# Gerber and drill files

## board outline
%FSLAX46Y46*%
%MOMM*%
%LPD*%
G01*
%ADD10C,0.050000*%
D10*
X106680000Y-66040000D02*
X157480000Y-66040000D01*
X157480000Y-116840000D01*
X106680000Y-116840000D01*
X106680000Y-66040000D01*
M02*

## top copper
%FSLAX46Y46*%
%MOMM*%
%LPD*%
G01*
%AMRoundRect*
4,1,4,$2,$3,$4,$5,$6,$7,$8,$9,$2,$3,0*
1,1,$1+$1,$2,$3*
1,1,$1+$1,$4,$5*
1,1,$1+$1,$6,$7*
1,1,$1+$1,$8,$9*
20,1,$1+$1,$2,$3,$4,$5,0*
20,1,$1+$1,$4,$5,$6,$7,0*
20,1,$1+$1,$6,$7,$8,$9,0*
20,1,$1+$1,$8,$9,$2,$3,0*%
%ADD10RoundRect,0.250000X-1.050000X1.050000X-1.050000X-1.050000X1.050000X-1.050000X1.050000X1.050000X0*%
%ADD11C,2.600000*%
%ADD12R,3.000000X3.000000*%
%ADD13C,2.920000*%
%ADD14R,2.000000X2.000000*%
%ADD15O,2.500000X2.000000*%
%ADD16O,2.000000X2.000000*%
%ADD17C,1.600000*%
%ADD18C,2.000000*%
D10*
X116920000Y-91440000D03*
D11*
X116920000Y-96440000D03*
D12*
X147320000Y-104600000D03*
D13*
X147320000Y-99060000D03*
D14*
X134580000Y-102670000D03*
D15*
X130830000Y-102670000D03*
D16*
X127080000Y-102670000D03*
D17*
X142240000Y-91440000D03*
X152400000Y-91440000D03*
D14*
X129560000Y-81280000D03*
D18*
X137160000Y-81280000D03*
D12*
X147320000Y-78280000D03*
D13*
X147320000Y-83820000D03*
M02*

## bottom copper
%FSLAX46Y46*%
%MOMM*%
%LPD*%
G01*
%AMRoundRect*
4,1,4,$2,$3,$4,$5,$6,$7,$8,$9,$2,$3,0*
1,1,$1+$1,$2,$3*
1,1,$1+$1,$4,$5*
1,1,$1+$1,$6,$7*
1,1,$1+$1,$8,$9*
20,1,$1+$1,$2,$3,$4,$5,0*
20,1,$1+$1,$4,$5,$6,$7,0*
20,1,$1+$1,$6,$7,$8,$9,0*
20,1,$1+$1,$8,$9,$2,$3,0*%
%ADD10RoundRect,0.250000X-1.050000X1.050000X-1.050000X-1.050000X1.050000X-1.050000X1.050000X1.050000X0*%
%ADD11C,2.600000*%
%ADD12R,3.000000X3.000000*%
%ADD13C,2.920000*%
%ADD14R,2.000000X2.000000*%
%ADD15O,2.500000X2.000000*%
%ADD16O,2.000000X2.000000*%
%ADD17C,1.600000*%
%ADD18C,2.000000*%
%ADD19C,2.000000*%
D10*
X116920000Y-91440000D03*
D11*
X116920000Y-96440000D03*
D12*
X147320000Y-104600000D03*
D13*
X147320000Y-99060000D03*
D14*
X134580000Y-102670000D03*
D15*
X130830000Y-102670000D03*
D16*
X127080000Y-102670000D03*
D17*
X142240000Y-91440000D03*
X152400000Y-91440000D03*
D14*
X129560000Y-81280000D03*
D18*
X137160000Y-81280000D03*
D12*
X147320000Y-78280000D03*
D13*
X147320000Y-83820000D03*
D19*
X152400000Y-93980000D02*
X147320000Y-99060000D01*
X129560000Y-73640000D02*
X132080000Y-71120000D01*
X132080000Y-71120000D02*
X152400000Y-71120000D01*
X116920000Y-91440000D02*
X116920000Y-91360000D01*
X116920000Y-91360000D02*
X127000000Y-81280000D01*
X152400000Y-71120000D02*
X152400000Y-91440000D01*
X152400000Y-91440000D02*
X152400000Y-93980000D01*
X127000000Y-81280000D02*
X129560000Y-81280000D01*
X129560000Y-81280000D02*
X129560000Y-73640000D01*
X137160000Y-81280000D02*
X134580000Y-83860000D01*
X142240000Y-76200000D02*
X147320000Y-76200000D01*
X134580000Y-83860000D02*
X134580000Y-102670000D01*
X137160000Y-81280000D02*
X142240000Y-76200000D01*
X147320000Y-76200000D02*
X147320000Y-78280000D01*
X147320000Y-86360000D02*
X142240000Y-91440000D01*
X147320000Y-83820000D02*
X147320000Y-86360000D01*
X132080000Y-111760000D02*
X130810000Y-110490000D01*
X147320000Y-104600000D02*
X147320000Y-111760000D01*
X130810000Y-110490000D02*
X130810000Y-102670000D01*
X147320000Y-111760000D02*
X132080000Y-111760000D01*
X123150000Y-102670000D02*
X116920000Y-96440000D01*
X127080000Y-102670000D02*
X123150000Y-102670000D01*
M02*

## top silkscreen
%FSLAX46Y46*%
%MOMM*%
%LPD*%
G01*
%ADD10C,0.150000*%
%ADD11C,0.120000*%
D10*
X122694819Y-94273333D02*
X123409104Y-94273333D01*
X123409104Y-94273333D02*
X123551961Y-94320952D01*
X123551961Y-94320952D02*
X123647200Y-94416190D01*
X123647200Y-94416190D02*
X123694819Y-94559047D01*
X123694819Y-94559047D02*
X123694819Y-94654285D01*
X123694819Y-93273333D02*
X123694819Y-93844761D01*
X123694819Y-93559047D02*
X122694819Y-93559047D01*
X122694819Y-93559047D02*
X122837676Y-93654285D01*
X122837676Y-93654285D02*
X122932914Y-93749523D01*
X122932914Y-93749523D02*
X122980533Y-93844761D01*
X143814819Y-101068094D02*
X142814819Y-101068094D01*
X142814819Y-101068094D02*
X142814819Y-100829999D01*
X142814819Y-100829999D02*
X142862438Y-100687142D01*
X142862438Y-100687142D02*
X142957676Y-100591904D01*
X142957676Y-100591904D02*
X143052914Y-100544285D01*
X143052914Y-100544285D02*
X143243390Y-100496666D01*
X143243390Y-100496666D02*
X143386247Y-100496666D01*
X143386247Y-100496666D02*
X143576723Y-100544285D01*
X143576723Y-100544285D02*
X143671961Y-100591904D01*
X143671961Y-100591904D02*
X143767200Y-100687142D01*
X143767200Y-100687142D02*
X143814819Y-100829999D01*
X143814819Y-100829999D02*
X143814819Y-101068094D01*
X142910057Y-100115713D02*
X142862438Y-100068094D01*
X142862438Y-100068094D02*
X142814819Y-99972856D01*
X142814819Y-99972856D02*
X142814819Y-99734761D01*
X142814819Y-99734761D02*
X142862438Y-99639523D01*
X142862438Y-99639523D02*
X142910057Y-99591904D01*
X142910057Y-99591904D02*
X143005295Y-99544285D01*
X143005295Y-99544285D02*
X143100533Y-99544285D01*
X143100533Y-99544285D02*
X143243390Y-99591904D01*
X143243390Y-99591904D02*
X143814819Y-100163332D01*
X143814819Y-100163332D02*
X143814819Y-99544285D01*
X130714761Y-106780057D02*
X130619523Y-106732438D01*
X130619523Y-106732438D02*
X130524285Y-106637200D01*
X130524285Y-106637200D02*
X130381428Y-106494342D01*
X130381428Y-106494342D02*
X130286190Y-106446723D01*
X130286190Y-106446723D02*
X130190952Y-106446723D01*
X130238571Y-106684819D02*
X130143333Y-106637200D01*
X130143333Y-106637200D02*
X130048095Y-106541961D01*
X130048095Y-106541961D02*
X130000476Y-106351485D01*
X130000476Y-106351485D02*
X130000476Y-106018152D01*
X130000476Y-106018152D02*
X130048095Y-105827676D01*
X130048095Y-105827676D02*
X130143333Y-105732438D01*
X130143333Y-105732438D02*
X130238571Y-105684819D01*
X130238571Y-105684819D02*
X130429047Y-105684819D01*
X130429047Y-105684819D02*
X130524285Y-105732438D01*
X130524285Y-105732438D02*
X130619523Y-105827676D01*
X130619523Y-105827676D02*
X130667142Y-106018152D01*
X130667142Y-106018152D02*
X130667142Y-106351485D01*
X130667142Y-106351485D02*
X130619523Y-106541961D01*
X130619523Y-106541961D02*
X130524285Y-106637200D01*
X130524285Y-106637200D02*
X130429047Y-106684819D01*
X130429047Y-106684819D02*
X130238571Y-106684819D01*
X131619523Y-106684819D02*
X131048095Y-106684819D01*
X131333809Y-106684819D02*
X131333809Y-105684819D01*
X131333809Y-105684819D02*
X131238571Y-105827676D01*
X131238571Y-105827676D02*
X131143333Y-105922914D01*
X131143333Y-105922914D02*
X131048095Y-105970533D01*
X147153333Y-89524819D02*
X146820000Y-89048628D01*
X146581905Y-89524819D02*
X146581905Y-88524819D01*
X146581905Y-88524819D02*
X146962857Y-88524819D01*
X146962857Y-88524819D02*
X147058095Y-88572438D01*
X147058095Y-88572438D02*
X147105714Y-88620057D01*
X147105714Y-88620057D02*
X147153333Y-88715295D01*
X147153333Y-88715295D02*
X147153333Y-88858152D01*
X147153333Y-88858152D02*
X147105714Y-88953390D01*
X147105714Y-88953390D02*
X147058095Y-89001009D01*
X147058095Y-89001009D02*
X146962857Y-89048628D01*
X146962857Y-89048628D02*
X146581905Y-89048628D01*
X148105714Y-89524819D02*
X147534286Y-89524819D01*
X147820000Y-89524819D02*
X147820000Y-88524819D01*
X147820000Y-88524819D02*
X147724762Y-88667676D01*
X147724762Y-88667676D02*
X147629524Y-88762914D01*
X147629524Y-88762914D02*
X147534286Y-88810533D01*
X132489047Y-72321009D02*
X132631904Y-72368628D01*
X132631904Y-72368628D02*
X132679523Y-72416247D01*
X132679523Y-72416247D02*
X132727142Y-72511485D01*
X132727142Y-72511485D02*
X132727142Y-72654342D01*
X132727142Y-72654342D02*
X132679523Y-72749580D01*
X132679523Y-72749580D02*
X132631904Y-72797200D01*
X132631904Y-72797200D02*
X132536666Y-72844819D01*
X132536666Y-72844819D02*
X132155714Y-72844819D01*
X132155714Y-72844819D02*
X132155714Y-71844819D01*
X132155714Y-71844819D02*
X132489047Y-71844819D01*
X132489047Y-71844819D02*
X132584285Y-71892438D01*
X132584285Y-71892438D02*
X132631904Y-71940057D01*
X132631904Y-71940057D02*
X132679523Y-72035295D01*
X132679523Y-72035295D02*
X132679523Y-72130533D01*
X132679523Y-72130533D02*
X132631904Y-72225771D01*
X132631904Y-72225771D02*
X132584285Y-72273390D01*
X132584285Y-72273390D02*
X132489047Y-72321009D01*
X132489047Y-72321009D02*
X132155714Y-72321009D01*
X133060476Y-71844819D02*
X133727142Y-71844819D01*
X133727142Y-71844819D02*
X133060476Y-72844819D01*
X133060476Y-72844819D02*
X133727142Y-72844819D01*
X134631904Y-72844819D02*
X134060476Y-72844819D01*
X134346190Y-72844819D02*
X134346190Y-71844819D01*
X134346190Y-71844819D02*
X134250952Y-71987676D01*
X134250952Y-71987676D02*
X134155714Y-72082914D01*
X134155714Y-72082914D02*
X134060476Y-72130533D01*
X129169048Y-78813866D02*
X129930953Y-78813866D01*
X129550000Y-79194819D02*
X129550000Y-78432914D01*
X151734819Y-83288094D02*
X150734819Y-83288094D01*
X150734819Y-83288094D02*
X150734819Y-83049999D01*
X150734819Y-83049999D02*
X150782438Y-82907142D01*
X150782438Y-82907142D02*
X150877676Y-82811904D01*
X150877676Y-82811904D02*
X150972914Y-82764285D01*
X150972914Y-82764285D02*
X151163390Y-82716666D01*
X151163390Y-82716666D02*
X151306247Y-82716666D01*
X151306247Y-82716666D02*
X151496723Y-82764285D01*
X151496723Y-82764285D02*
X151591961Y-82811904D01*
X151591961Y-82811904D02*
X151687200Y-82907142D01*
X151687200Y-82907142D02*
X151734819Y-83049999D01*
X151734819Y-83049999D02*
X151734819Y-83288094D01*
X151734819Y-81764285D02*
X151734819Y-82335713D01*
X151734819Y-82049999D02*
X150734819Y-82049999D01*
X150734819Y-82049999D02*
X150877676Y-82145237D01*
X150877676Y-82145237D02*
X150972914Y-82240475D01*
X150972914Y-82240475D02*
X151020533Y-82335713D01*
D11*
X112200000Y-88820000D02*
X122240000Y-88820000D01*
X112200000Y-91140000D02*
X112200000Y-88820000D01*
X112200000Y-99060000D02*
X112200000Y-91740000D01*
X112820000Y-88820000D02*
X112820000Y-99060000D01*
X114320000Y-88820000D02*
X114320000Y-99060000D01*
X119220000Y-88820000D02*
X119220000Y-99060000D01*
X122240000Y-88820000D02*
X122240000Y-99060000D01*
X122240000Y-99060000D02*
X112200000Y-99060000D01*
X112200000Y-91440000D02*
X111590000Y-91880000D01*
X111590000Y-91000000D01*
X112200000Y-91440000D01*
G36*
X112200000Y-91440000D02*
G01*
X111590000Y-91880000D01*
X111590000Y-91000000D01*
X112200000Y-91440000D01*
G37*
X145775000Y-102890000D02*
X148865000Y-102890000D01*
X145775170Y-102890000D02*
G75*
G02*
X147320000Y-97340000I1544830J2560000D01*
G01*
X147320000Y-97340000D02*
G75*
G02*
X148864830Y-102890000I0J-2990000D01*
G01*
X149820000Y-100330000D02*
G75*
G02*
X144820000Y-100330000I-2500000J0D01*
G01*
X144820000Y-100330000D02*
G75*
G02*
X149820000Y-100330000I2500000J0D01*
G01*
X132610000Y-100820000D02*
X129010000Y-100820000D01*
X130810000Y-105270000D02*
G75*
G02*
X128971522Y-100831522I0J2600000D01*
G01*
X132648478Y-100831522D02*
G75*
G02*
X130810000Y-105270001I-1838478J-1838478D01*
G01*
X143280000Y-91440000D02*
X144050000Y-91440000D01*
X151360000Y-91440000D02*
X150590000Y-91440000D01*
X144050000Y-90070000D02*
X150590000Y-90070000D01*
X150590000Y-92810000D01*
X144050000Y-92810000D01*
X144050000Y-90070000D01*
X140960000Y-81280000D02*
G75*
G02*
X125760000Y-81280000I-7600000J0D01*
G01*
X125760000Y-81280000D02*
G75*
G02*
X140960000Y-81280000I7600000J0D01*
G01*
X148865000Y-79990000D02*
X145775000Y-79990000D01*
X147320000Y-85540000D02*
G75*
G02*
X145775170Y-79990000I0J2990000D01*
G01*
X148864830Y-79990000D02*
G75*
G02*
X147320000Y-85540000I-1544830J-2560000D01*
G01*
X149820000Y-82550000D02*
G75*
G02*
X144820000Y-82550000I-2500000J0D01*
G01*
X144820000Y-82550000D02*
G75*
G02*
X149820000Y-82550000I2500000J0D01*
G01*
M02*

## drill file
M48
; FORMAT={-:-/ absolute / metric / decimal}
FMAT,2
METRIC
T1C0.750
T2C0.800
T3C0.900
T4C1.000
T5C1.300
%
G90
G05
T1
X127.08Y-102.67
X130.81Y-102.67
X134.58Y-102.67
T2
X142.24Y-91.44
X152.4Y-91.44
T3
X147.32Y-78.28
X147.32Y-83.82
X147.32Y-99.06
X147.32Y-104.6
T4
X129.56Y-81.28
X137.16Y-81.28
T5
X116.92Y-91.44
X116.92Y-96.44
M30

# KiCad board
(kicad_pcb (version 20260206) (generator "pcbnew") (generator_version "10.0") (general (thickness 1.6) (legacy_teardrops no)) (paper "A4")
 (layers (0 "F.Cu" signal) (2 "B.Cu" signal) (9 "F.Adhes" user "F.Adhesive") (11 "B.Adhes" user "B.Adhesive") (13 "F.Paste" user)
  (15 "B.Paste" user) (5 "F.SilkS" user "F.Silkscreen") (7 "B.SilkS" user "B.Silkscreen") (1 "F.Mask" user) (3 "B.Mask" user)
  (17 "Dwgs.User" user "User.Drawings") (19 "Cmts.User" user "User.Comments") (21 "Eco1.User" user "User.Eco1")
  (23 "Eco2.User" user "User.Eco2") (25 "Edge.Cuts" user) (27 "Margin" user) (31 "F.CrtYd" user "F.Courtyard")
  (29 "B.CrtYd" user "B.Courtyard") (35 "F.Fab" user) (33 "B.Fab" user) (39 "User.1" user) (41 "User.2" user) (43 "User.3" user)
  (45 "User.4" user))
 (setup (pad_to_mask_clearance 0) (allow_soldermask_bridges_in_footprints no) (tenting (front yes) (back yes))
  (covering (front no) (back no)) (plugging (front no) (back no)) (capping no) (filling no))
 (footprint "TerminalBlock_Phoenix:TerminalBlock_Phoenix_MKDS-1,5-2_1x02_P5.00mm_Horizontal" (layer "F.Cu") (at 116.92 91.44 -90)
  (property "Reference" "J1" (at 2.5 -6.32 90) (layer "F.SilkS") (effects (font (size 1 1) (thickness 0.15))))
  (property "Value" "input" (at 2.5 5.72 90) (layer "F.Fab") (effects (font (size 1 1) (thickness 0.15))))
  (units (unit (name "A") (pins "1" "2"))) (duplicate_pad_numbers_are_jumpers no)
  (fp_line (start -2.62 4.72) (end -2.62 -5.32) (stroke (width 0.12) (type solid)) (layer "F.SilkS"))
  (fp_line (start -0.3 4.72) (end -2.62 4.72) (stroke (width 0.12) (type solid)) (layer "F.SilkS"))
  (fp_line (start 7.62 4.72) (end 0.3 4.72) (stroke (width 0.12) (type solid)) (layer "F.SilkS"))
  (fp_line (start -2.62 4.1) (end 7.62 4.1) (stroke (width 0.12) (type solid)) (layer "F.SilkS"))
  (fp_line (start -2.62 2.6) (end 7.62 2.6) (stroke (width 0.12) (type solid)) (layer "F.SilkS"))
  (fp_line (start -2.62 -2.3) (end 7.62 -2.3) (stroke (width 0.12) (type solid)) (layer "F.SilkS"))
  (fp_line (start -2.62 -5.32) (end 7.62 -5.32) (stroke (width 0.12) (type solid)) (layer "F.SilkS"))
  (fp_line (start 7.62 -5.32) (end 7.62 4.72) (stroke (width 0.12) (type solid)) (layer "F.SilkS"))
  (fp_poly (pts (xy 0 4.72) (xy 0.44 5.33) (xy -0.44 5.33)) (stroke (width 0.12) (type solid)) (fill yes) (layer "F.SilkS"))
  (pad "1" thru_hole roundrect (at 0 0 270) (size 2.6 2.6) (drill 1.3) (layers "*.Cu" "*.Mask") (remove_unused_layers no)
   (roundrect_rratio 0.096154) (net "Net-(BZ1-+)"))
  (pad "2" thru_hole circle (at 5 0 270) (size 2.6 2.6) (drill 1.3) (layers "*.Cu" "*.Mask") (remove_unused_layers no)
   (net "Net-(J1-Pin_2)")))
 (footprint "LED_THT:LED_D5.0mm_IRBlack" (layer "F.Cu") (at 147.32 101.6 90)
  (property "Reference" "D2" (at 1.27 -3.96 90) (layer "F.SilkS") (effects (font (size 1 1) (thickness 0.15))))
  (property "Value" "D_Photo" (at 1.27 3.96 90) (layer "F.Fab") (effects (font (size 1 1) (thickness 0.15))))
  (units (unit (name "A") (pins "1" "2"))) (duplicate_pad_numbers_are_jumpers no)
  (fp_line (start -1.29 -1.545) (end -1.29 1.545) (stroke (width 0.12) (type solid)) (layer "F.SilkS"))
  (fp_arc (start -1.29 -1.54483) (mid 2.071779 -2.880495) (end 4.26 0) (stroke (width 0.12) (type solid)) (layer "F.SilkS"))
  (fp_arc (start 4.26 0) (mid 2.071779 2.880495) (end -1.29 1.54483) (stroke (width 0.12) (type solid)) (layer "F.SilkS"))
  (fp_circle (center 1.27 0) (end 3.77 0) (stroke (width 0.12) (type solid)) (fill no) (layer "F.SilkS"))
  (pad "1" thru_hole rect (at -3 0 90) (size 3 3) (drill 0.9) (layers "*.Cu" "*.Mask") (remove_unused_layers no) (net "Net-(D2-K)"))
  (pad "2" thru_hole circle (at 2.54 0 90) (size 2.92 2.92) (drill 0.9) (layers "*.Cu" "*.Mask") (remove_unused_layers no)
   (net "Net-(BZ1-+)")))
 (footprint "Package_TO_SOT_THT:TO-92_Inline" (layer "F.Cu") (at 132.08 102.67 180)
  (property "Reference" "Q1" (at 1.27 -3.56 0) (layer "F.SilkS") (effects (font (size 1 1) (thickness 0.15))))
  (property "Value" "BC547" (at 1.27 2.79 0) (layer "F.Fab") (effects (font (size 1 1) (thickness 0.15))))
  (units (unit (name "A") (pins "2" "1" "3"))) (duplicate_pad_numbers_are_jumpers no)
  (fp_line (start -0.53 1.85) (end 3.07 1.85) (stroke (width 0.12) (type solid)) (layer "F.SilkS"))
  (fp_arc (start 1.27 -2.6) (mid 3.672087 -0.994977) (end 3.108478 1.838478) (stroke (width 0.12) (type solid)) (layer "F.SilkS"))
  (fp_arc (start -0.568478 1.838478) (mid -1.132087 -0.994977) (end 1.27 -2.6) (stroke (width 0.12) (type solid)) (layer "F.SilkS"))
  (pad "1" thru_hole rect (at -2.5 0 180) (size 2 2) (drill 0.75) (layers "*.Cu" "*.Mask") (remove_unused_layers no) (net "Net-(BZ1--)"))
  (pad "2" thru_hole oval (at 1.27 0 180) (size 2.5 2) (drill 0.75 (offset -0.02 0)) (layers "*.Cu" "*.Mask") (remove_unused_layers no)
   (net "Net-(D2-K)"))
  (pad "3" thru_hole oval (at 5 0 180) (size 2 2) (drill 0.75) (layers "*.Cu" "*.Mask") (remove_unused_layers no) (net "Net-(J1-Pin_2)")))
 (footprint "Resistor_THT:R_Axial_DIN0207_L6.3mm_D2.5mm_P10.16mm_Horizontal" (layer "F.Cu") (at 142.24 91.44)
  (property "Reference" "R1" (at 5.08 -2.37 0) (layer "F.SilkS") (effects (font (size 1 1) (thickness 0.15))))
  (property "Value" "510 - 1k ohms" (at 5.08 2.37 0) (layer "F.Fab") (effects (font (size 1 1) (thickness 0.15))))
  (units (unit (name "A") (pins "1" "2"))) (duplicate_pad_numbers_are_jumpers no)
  (fp_line (start 1.04 0) (end 1.81 0) (stroke (width 0.12) (type solid)) (layer "F.SilkS"))
  (fp_line (start 9.12 0) (end 8.35 0) (stroke (width 0.12) (type solid)) (layer "F.SilkS"))
  (fp_rect (start 1.81 -1.37) (end 8.35 1.37) (stroke (width 0.12) (type solid)) (fill no) (layer "F.SilkS"))
  (pad "1" thru_hole circle (at 0 0) (size 1.6 1.6) (drill 0.8) (layers "*.Cu" "*.Mask") (remove_unused_layers no) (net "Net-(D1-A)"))
  (pad "2" thru_hole circle (at 10.16 0) (size 1.6 1.6) (drill 0.8) (layers "*.Cu" "*.Mask") (remove_unused_layers no) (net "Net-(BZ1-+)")))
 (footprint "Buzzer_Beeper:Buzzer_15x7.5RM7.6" (layer "F.Cu") (at 129.56 81.28)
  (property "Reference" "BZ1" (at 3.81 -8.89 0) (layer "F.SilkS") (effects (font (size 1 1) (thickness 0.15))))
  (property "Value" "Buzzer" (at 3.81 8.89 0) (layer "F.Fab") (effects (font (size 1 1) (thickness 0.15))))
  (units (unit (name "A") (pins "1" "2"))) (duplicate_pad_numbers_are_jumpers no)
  (fp_circle (center 3.8 0) (end 11.4 0) (stroke (width 0.12) (type solid)) (fill no) (layer "F.SilkS"))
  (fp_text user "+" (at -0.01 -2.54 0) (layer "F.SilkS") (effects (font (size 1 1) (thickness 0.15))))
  (pad "1" thru_hole rect (at 0 0) (size 2 2) (drill 1) (layers "*.Cu" "*.Mask") (remove_unused_layers no) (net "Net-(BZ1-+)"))
  (pad "2" thru_hole circle (at 7.6 0) (size 2 2) (drill 1) (layers "*.Cu" "*.Mask") (remove_unused_layers no) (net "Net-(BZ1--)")))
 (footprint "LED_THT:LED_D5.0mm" (layer "F.Cu") (at 147.32 81.28 -90)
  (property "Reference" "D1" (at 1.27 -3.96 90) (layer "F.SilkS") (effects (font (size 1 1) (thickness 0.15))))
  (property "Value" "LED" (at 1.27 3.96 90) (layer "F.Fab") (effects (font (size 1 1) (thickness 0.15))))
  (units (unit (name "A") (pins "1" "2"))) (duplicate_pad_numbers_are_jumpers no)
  (fp_line (start -1.29 -1.545) (end -1.29 1.545) (stroke (width 0.12) (type solid)) (layer "F.SilkS"))
  (fp_arc (start 4.26 0) (mid 2.071779 2.880495) (end -1.29 1.54483) (stroke (width 0.12) (type solid)) (layer "F.SilkS"))
  (fp_arc (start -1.29 -1.54483) (mid 2.071779 -2.880495) (end 4.26 0) (stroke (width 0.12) (type solid)) (layer "F.SilkS"))
  (fp_circle (center 1.27 0) (end 3.77 0) (stroke (width 0.12) (type solid)) (fill no) (layer "F.SilkS"))
  (pad "1" thru_hole rect (at -3 0 270) (size 3 3) (drill 0.9) (layers "*.Cu" "*.Mask") (remove_unused_layers no) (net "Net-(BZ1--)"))
  (pad "2" thru_hole circle (at 2.54 0 270) (size 2.92 2.92) (drill 0.9) (layers "*.Cu" "*.Mask") (remove_unused_layers no)
   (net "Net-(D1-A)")))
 (gr_rect (start 106.68 66.04) (end 157.48 116.84) (stroke (width 0.05) (type default)) (fill no) (layer "Edge.Cuts"))
 (segment (start 152.4 93.98) (end 147.32 99.06) (width 2) (layer "B.Cu") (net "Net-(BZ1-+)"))
 (segment (start 129.56 73.64) (end 132.08 71.12) (width 2) (layer "B.Cu") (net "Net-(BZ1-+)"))
 (segment (start 132.08 71.12) (end 152.4 71.12) (width 2) (layer "B.Cu") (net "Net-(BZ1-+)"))
 (segment (start 116.92 91.44) (end 116.92 91.36) (width 2) (layer "B.Cu") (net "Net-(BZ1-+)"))
 (segment (start 116.92 91.36) (end 127 81.28) (width 2) (layer "B.Cu") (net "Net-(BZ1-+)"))
 (segment (start 152.4 71.12) (end 152.4 91.44) (width 2) (layer "B.Cu") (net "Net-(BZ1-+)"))
 (segment (start 152.4 91.44) (end 152.4 93.98) (width 2) (layer "B.Cu") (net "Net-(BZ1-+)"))
 (segment (start 127 81.28) (end 129.56 81.28) (width 2) (layer "B.Cu") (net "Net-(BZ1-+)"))
 (segment (start 129.56 81.28) (end 129.56 73.64) (width 2) (layer "B.Cu") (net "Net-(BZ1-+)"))
 (segment (start 137.16 81.28) (end 134.58 83.86) (width 2) (layer "B.Cu") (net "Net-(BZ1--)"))
 (segment (start 142.24 76.2) (end 147.32 76.2) (width 2) (layer "B.Cu") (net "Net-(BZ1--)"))
 (segment (start 134.58 83.86) (end 134.58 102.67) (width 2) (layer "B.Cu") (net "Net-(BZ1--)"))
 (segment (start 137.16 81.28) (end 142.24 76.2) (width 2) (layer "B.Cu") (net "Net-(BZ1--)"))
 (segment (start 147.32 76.2) (end 147.32 78.28) (width 2) (layer "B.Cu") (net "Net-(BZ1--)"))
 (segment (start 147.32 86.36) (end 142.24 91.44) (width 2) (layer "B.Cu") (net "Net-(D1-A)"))
 (segment (start 147.32 83.82) (end 147.32 86.36) (width 2) (layer "B.Cu") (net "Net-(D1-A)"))
 (segment (start 132.08 111.76) (end 130.81 110.49) (width 2) (layer "B.Cu") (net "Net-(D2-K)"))
 (segment (start 147.32 104.6) (end 147.32 111.76) (width 2) (layer "B.Cu") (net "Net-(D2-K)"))
 (segment (start 130.81 110.49) (end 130.81 102.67) (width 2) (layer "B.Cu") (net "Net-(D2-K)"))
 (segment (start 147.32 111.76) (end 132.08 111.76) (width 2) (layer "B.Cu") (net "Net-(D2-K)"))
 (segment (start 123.15 102.67) (end 116.92 96.44) (width 2) (layer "B.Cu") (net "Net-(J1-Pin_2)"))
 (segment (start 127.08 102.67) (end 123.15 102.67) (width 2) (layer "B.Cu") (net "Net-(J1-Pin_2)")))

